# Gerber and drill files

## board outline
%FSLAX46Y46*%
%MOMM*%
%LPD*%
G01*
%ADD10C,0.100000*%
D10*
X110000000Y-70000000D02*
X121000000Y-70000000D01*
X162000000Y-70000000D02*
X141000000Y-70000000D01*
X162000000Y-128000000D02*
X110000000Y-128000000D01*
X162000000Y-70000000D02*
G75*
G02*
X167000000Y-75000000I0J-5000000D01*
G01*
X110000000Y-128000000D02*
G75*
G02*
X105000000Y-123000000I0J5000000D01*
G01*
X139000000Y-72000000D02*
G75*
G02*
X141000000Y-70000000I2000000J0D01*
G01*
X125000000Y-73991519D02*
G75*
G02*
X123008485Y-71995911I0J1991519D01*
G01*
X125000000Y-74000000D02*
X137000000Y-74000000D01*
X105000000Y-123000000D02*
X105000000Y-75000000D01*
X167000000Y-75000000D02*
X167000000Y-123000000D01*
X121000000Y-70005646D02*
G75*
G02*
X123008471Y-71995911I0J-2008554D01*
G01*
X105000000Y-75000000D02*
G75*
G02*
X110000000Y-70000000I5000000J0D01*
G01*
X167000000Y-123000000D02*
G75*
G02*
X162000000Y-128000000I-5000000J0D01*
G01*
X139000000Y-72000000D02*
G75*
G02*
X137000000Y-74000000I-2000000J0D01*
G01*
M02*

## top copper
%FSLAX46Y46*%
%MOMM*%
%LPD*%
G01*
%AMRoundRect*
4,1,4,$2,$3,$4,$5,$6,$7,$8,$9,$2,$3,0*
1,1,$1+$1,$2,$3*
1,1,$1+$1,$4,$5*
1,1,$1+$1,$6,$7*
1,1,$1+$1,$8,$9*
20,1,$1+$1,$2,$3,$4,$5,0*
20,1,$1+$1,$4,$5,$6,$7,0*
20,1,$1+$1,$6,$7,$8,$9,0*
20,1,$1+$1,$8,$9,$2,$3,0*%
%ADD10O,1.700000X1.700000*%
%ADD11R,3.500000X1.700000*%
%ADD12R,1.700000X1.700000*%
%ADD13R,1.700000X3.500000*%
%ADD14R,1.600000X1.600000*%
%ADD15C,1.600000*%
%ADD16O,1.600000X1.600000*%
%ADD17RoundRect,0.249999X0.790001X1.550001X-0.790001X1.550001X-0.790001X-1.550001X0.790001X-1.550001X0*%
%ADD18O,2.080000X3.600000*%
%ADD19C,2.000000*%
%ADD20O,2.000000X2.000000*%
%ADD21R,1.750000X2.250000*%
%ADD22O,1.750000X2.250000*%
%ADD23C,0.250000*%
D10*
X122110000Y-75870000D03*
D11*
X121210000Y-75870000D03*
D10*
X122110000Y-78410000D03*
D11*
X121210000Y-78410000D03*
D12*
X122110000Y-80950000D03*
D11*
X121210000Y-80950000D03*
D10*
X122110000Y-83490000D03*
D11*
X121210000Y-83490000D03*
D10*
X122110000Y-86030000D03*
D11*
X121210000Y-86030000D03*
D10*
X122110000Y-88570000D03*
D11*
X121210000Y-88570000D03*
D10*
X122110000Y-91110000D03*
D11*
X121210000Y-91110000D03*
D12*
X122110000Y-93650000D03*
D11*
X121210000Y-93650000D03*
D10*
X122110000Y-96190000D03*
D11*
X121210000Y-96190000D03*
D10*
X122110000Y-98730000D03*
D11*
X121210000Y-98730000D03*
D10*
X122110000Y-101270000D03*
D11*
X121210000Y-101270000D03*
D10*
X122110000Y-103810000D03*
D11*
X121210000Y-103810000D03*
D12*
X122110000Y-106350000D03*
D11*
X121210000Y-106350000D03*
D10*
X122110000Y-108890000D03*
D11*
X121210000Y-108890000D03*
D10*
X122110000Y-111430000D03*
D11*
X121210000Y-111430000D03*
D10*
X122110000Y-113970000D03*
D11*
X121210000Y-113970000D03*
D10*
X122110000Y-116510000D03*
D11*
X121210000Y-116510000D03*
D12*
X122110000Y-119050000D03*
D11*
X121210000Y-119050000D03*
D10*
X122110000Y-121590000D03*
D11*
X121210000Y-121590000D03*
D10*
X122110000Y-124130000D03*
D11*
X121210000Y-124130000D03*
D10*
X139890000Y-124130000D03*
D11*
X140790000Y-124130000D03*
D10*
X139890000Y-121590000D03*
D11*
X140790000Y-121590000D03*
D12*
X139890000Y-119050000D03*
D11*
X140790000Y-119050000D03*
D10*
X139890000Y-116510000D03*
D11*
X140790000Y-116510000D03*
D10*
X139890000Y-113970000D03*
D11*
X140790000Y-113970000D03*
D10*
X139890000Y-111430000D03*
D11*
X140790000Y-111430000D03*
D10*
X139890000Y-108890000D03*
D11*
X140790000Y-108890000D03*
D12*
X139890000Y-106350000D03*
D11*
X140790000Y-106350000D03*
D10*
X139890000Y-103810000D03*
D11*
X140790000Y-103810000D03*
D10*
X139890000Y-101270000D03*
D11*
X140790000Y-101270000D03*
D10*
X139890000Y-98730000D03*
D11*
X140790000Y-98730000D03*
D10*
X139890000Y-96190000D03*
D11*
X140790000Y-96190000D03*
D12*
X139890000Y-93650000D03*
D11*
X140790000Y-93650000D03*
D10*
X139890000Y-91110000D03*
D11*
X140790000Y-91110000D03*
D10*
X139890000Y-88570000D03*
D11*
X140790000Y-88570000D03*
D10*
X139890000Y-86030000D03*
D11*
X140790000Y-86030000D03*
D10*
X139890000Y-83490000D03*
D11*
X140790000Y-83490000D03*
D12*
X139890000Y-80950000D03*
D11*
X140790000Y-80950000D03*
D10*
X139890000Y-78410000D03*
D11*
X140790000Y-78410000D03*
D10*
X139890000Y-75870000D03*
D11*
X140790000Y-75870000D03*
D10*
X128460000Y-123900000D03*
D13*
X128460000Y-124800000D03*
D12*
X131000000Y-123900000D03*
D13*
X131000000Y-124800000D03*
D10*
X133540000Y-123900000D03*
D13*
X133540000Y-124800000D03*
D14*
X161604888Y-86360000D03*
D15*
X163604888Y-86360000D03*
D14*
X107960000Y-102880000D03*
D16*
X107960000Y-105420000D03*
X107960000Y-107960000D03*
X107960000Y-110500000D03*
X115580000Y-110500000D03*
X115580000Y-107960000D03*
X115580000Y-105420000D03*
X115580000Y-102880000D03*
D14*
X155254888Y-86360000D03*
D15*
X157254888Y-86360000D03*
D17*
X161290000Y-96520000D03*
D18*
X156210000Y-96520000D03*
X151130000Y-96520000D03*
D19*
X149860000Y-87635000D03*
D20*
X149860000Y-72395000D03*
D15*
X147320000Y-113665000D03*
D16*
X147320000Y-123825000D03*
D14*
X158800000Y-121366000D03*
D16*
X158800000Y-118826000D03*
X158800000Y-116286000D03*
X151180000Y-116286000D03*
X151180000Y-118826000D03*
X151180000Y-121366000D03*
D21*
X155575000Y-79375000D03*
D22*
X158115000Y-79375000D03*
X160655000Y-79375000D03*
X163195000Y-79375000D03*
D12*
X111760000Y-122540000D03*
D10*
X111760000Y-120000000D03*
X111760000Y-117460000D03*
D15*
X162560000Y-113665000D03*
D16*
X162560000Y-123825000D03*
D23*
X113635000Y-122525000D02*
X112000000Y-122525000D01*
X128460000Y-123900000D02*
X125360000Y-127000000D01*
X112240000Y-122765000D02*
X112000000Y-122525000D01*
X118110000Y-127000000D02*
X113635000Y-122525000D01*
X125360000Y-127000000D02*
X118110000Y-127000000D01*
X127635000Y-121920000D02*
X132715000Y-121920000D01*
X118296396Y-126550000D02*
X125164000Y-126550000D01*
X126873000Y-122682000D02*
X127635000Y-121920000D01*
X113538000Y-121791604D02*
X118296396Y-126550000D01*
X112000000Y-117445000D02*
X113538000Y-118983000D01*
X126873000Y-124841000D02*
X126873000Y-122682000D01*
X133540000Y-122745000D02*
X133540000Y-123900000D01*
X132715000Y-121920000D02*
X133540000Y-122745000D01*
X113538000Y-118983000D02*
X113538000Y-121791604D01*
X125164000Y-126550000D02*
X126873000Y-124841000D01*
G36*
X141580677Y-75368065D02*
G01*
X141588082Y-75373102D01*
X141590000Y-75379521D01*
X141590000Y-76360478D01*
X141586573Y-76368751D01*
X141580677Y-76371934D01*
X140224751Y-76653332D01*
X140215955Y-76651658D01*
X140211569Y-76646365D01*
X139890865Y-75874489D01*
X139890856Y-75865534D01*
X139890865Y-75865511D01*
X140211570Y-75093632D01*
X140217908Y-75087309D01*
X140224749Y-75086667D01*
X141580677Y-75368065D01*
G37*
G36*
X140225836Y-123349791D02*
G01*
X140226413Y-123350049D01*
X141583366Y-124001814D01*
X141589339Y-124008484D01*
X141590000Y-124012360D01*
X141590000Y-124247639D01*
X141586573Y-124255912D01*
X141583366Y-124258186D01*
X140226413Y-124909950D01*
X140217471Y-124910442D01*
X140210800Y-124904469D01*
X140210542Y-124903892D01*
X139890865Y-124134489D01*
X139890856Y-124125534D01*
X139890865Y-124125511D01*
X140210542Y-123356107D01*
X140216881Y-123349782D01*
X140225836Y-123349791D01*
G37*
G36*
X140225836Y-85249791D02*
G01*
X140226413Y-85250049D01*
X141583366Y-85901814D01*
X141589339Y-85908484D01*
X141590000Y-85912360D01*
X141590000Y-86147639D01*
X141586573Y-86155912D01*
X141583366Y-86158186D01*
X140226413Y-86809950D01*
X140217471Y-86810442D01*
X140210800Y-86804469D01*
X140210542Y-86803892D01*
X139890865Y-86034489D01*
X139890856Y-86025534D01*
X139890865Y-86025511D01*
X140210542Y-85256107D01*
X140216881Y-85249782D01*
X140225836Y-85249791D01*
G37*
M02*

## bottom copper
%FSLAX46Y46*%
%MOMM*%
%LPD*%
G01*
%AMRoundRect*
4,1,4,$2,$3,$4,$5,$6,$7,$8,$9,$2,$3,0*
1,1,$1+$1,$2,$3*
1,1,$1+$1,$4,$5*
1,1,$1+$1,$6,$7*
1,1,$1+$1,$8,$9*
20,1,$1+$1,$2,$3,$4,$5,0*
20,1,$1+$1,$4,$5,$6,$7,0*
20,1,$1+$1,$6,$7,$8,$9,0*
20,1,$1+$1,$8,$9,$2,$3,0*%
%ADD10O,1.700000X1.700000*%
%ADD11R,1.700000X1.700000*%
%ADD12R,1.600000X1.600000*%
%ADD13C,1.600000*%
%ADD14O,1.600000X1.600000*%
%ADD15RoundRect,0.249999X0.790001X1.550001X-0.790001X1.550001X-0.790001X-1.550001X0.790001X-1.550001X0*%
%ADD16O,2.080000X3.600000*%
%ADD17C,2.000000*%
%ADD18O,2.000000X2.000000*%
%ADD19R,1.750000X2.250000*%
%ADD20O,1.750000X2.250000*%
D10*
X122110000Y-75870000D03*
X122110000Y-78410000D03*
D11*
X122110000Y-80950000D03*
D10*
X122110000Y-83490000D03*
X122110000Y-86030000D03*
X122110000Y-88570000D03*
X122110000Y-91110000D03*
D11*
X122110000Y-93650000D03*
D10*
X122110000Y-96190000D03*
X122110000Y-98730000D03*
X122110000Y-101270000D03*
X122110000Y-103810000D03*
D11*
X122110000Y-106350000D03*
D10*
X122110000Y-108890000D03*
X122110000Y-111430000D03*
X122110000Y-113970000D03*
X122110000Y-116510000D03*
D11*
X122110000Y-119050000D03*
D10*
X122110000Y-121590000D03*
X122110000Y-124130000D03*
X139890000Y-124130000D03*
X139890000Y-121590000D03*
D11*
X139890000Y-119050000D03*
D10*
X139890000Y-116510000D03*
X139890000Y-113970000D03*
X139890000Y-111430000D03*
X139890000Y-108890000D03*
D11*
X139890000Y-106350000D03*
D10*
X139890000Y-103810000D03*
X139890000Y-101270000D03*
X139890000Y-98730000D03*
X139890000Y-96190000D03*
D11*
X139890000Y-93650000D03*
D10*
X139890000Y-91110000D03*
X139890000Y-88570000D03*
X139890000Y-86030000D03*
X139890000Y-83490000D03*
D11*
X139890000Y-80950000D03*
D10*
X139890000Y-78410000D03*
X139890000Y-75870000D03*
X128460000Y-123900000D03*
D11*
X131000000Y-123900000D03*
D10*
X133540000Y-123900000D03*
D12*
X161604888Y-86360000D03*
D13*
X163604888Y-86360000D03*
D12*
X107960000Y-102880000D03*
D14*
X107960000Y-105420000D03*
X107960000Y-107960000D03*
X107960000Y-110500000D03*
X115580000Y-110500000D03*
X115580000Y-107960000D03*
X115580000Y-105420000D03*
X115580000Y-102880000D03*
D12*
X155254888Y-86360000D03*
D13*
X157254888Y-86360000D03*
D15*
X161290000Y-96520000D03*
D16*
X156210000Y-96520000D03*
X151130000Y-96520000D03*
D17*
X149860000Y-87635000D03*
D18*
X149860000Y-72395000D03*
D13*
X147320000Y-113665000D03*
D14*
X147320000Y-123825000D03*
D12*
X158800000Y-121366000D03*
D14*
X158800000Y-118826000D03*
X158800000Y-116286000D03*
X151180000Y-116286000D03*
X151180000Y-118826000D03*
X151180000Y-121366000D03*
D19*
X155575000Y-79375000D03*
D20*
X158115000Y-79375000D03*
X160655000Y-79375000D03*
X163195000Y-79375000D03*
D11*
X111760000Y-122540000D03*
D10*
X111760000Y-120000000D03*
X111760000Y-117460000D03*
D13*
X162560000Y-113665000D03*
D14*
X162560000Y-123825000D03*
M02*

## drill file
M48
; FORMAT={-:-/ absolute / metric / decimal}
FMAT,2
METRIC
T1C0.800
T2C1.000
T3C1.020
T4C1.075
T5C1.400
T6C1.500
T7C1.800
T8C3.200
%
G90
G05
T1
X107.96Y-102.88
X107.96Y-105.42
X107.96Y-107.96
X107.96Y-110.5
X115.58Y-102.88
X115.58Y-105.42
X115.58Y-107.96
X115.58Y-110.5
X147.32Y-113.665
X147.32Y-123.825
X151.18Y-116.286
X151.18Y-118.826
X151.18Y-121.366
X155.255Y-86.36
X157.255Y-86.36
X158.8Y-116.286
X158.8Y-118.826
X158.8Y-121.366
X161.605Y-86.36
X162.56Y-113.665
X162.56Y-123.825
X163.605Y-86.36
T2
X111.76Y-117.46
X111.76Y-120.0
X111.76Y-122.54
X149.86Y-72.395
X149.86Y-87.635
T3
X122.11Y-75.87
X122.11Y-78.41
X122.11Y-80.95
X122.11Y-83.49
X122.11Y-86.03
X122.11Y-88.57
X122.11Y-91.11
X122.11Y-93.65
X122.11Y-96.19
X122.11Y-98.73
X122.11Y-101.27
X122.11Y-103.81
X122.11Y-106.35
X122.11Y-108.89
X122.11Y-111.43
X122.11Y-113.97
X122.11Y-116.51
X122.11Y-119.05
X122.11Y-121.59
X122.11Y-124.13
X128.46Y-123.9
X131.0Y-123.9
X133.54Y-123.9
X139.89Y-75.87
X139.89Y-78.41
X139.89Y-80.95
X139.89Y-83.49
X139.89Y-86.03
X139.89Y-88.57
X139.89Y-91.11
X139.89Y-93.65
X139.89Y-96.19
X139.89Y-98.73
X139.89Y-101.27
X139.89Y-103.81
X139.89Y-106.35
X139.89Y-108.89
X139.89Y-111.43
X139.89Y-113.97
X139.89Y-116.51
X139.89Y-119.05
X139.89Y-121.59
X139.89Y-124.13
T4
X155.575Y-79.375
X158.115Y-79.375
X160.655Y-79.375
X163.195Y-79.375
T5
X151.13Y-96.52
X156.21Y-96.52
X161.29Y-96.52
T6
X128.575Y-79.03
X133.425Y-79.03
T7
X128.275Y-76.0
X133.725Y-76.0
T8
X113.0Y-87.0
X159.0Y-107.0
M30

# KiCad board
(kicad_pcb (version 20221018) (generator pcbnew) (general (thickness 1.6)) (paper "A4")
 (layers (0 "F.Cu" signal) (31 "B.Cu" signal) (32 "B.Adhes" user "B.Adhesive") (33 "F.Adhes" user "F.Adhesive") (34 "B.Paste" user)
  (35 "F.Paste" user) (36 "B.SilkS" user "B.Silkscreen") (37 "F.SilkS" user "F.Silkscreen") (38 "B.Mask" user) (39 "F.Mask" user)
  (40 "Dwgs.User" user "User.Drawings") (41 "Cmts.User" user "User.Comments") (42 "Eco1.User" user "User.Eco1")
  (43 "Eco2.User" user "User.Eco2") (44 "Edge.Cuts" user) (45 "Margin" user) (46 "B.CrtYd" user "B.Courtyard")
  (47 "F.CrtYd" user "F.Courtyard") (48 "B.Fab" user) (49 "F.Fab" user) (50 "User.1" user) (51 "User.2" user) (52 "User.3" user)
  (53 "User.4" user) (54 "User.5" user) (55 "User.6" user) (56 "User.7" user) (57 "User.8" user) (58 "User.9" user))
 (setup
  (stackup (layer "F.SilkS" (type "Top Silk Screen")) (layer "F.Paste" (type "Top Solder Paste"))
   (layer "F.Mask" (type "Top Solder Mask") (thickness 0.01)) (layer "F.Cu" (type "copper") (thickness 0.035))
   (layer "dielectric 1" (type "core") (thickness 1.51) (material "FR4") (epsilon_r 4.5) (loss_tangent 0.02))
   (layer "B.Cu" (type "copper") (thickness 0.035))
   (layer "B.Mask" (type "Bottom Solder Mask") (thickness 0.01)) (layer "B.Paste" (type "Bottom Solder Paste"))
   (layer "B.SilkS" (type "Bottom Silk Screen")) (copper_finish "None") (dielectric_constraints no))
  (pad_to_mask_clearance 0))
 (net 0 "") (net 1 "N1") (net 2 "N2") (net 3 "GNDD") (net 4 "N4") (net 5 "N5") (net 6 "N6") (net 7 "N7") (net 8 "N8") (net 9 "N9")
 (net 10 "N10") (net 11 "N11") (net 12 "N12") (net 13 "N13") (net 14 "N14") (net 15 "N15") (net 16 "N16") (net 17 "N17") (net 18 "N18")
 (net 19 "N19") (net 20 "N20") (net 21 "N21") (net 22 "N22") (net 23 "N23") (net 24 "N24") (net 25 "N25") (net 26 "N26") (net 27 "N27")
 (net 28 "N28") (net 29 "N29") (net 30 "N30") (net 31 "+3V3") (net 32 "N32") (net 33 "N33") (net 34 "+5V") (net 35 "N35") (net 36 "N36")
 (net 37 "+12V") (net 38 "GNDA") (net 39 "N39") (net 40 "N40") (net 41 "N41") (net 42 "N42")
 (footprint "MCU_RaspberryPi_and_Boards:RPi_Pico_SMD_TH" (layer "F.Cu") (at 131 100)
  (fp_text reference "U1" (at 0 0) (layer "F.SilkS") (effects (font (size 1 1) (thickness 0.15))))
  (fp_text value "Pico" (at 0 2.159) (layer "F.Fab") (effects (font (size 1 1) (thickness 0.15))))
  (pad "" np_thru_hole oval (at -2.725 -24) (size 1.8 1.8) (drill 1.8) (layers "*.Cu" "*.Mask"))
  (pad "" np_thru_hole oval (at -2.425 -20.97) (size 1.5 1.5) (drill 1.5) (layers "*.Cu" "*.Mask"))
  (pad "" np_thru_hole oval (at 2.425 -20.97) (size 1.5 1.5) (drill 1.5) (layers "*.Cu" "*.Mask"))
  (pad "" np_thru_hole oval (at 2.725 -24) (size 1.8 1.8) (drill 1.8) (layers "*.Cu" "*.Mask"))
  (pad "1" thru_hole oval (at -8.89 -24.13) (size 1.7 1.7) (drill 1.02) (layers "*.Cu" "*.Mask") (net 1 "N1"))
  (pad "1" smd rect (at -8.89 -24.13) (size 3.5 1.7) (drill (offset -0.9 0)) (layers "F.Cu" "F.Mask") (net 1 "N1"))
  (pad "2" thru_hole oval (at -8.89 -21.59) (size 1.7 1.7) (drill 1.02) (layers "*.Cu" "*.Mask") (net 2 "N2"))
  (pad "2" smd rect (at -8.89 -21.59) (size 3.5 1.7) (drill (offset -0.9 0)) (layers "F.Cu" "F.Mask") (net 2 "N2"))
  (pad "3" thru_hole rect (at -8.89 -19.05) (size 1.7 1.7) (drill 1.02) (layers "*.Cu" "*.Mask") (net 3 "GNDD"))
  (pad "3" smd rect (at -8.89 -19.05) (size 3.5 1.7) (drill (offset -0.9 0)) (layers "F.Cu" "F.Mask") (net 3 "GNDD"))
  (pad "4" thru_hole oval (at -8.89 -16.51) (size 1.7 1.7) (drill 1.02) (layers "*.Cu" "*.Mask") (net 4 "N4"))
  (pad "4" smd rect (at -8.89 -16.51) (size 3.5 1.7) (drill (offset -0.9 0)) (layers "F.Cu" "F.Mask") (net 4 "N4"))
  (pad "5" thru_hole oval (at -8.89 -13.97) (size 1.7 1.7) (drill 1.02) (layers "*.Cu" "*.Mask") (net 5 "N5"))
  (pad "5" smd rect (at -8.89 -13.97) (size 3.5 1.7) (drill (offset -0.9 0)) (layers "F.Cu" "F.Mask") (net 5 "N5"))
  (pad "6" thru_hole oval (at -8.89 -11.43) (size 1.7 1.7) (drill 1.02) (layers "*.Cu" "*.Mask") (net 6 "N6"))
  (pad "6" smd rect (at -8.89 -11.43) (size 3.5 1.7) (drill (offset -0.9 0)) (layers "F.Cu" "F.Mask") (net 6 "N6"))
  (pad "7" thru_hole oval (at -8.89 -8.89) (size 1.7 1.7) (drill 1.02) (layers "*.Cu" "*.Mask") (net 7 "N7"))
  (pad "7" smd rect (at -8.89 -8.89) (size 3.5 1.7) (drill (offset -0.9 0)) (layers "F.Cu" "F.Mask") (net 7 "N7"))
  (pad "8" thru_hole rect (at -8.89 -6.35) (size 1.7 1.7) (drill 1.02) (layers "*.Cu" "*.Mask") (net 3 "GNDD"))
  (pad "8" smd rect (at -8.89 -6.35) (size 3.5 1.7) (drill (offset -0.9 0)) (layers "F.Cu" "F.Mask") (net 3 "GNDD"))
  (pad "9" thru_hole oval (at -8.89 -3.81) (size 1.7 1.7) (drill 1.02) (layers "*.Cu" "*.Mask") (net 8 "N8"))
  (pad "9" smd rect (at -8.89 -3.81) (size 3.5 1.7) (drill (offset -0.9 0)) (layers "F.Cu" "F.Mask") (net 8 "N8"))
  (pad "10" thru_hole oval (at -8.89 -1.27) (size 1.7 1.7) (drill 1.02) (layers "*.Cu" "*.Mask") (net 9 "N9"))
  (pad "10" smd rect (at -8.89 -1.27) (size 3.5 1.7) (drill (offset -0.9 0)) (layers "F.Cu" "F.Mask") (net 9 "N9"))
  (pad "11" thru_hole oval (at -8.89 1.27) (size 1.7 1.7) (drill 1.02) (layers "*.Cu" "*.Mask") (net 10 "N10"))
  (pad "11" smd rect (at -8.89 1.27) (size 3.5 1.7) (drill (offset -0.9 0)) (layers "F.Cu" "F.Mask") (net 10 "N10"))
  (pad "12" thru_hole oval (at -8.89 3.81) (size 1.7 1.7) (drill 1.02) (layers "*.Cu" "*.Mask") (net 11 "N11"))
  (pad "12" smd rect (at -8.89 3.81) (size 3.5 1.7) (drill (offset -0.9 0)) (layers "F.Cu" "F.Mask") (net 11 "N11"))
  (pad "13" thru_hole rect (at -8.89 6.35) (size 1.7 1.7) (drill 1.02) (layers "*.Cu" "*.Mask") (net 3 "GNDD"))
  (pad "13" smd rect (at -8.89 6.35) (size 3.5 1.7) (drill (offset -0.9 0)) (layers "F.Cu" "F.Mask") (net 3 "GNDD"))
  (pad "14" thru_hole oval (at -8.89 8.89) (size 1.7 1.7) (drill 1.02) (layers "*.Cu" "*.Mask") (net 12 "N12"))
  (pad "14" smd rect (at -8.89 8.89) (size 3.5 1.7) (drill (offset -0.9 0)) (layers "F.Cu" "F.Mask") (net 12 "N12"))
  (pad "15" thru_hole oval (at -8.89 11.43) (size 1.7 1.7) (drill 1.02) (layers "*.Cu" "*.Mask") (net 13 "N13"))
  (pad "15" smd rect (at -8.89 11.43) (size 3.5 1.7) (drill (offset -0.9 0)) (layers "F.Cu" "F.Mask") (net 13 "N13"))
  (pad "16" thru_hole oval (at -8.89 13.97) (size 1.7 1.7) (drill 1.02) (layers "*.Cu" "*.Mask") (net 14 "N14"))
  (pad "16" smd rect (at -8.89 13.97) (size 3.5 1.7) (drill (offset -0.9 0)) (layers "F.Cu" "F.Mask") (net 14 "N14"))
  (pad "17" thru_hole oval (at -8.89 16.51) (size 1.7 1.7) (drill 1.02) (layers "*.Cu" "*.Mask") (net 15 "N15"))
  (pad "17" smd rect (at -8.89 16.51) (size 3.5 1.7) (drill (offset -0.9 0)) (layers "F.Cu" "F.Mask") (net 15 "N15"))
  (pad "18" thru_hole rect (at -8.89 19.05) (size 1.7 1.7) (drill 1.02) (layers "*.Cu" "*.Mask") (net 3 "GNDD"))
  (pad "18" smd rect (at -8.89 19.05) (size 3.5 1.7) (drill (offset -0.9 0)) (layers "F.Cu" "F.Mask") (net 3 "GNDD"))
  (pad "19" thru_hole oval (at -8.89 21.59) (size 1.7 1.7) (drill 1.02) (layers "*.Cu" "*.Mask") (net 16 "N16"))
  (pad "19" smd rect (at -8.89 21.59) (size 3.5 1.7) (drill (offset -0.9 0)) (layers "F.Cu" "F.Mask") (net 16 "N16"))
  (pad "20" thru_hole oval (at -8.89 24.13) (size 1.7 1.7) (drill 1.02) (layers "*.Cu" "*.Mask") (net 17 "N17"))
  (pad "20" smd rect (at -8.89 24.13) (size 3.5 1.7) (drill (offset -0.9 0)) (layers "F.Cu" "F.Mask") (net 17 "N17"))
  (pad "21" thru_hole oval (at 8.89 24.13) (size 1.7 1.7) (drill 1.02) (layers "*.Cu" "*.Mask") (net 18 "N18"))
  (pad "21" smd rect (at 8.89 24.13) (size 3.5 1.7) (drill (offset 0.9 0)) (layers "F.Cu" "F.Mask") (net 18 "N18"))
  (pad "22" thru_hole oval (at 8.89 21.59) (size 1.7 1.7) (drill 1.02) (layers "*.Cu" "*.Mask") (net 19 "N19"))
  (pad "22" smd rect (at 8.89 21.59) (size 3.5 1.7) (drill (offset 0.9 0)) (layers "F.Cu" "F.Mask") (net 19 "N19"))
  (pad "23" thru_hole rect (at 8.89 19.05) (size 1.7 1.7) (drill 1.02) (layers "*.Cu" "*.Mask") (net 3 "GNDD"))
  (pad "23" smd rect (at 8.89 19.05) (size 3.5 1.7) (drill (offset 0.9 0)) (layers "F.Cu" "F.Mask") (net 3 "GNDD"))
  (pad "24" thru_hole oval (at 8.89 16.51) (size 1.7 1.7) (drill 1.02) (layers "*.Cu" "*.Mask") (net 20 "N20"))
  (pad "24" smd rect (at 8.89 16.51) (size 3.5 1.7) (drill (offset 0.9 0)) (layers "F.Cu" "F.Mask") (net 20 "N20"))
  (pad "25" thru_hole oval (at 8.89 13.97) (size 1.7 1.7) (drill 1.02) (layers "*.Cu" "*.Mask") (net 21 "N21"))
  (pad "25" smd rect (at 8.89 13.97) (size 3.5 1.7) (drill (offset 0.9 0)) (layers "F.Cu" "F.Mask") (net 21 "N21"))
  (pad "26" thru_hole oval (at 8.89 11.43) (size 1.7 1.7) (drill 1.02) (layers "*.Cu" "*.Mask") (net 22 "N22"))
  (pad "26" smd rect (at 8.89 11.43) (size 3.5 1.7) (drill (offset 0.9 0)) (layers "F.Cu" "F.Mask") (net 22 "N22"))
  (pad "27" thru_hole oval (at 8.89 8.89) (size 1.7 1.7) (drill 1.02) (layers "*.Cu" "*.Mask") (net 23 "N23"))
  (pad "27" smd rect (at 8.89 8.89) (size 3.5 1.7) (drill (offset 0.9 0)) (layers "F.Cu" "F.Mask") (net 23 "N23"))
  (pad "28" thru_hole rect (at 8.89 6.35) (size 1.7 1.7) (drill 1.02) (layers "*.Cu" "*.Mask") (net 3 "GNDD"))
  (pad "28" smd rect (at 8.89 6.35) (size 3.5 1.7) (drill (offset 0.9 0)) (layers "F.Cu" "F.Mask") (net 3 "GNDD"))
  (pad "29" thru_hole oval (at 8.89 3.81) (size 1.7 1.7) (drill 1.02) (layers "*.Cu" "*.Mask") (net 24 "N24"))
  (pad "29" smd rect (at 8.89 3.81) (size 3.5 1.7) (drill (offset 0.9 0)) (layers "F.Cu" "F.Mask") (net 24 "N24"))
  (pad "30" thru_hole oval (at 8.89 1.27) (size 1.7 1.7) (drill 1.02) (layers "*.Cu" "*.Mask") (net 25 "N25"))
  (pad "30" smd rect (at 8.89 1.27) (size 3.5 1.7) (drill (offset 0.9 0)) (layers "F.Cu" "F.Mask") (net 25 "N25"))
  (pad "31" thru_hole oval (at 8.89 -1.27) (size 1.7 1.7) (drill 1.02) (layers "*.Cu" "*.Mask") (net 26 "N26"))
  (pad "31" smd rect (at 8.89 -1.27) (size 3.5 1.7) (drill (offset 0.9 0)) (layers "F.Cu" "F.Mask") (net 26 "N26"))
  (pad "32" thru_hole oval (at 8.89 -3.81) (size 1.7 1.7) (drill 1.02) (layers "*.Cu" "*.Mask") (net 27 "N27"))
  (pad "32" smd rect (at 8.89 -3.81) (size 3.5 1.7) (drill (offset 0.9 0)) (layers "F.Cu" "F.Mask") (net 27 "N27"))
  (pad "33" thru_hole rect (at 8.89 -6.35) (size 1.7 1.7) (drill 1.02) (layers "*.Cu" "*.Mask") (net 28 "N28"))
  (pad "33" smd rect (at 8.89 -6.35) (size 3.5 1.7) (drill (offset 0.9 0)) (layers "F.Cu" "F.Mask") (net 28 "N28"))
  (pad "34" thru_hole oval (at 8.89 -8.89) (size 1.7 1.7) (drill 1.02) (layers "*.Cu" "*.Mask") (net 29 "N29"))
  (pad "34" smd rect (at 8.89 -8.89) (size 3.5 1.7) (drill (offset 0.9 0)) (layers "F.Cu" "F.Mask") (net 29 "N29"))
  (pad "35" thru_hole oval (at 8.89 -11.43) (size 1.7 1.7) (drill 1.02) (layers "*.Cu" "*.Mask") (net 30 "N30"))
  (pad "35" smd rect (at 8.89 -11.43) (size 3.5 1.7) (drill (offset 0.9 0)) (layers "F.Cu" "F.Mask") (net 30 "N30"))
  (pad "36" thru_hole oval (at 8.89 -13.97) (size 1.7 1.7) (drill 1.02) (layers "*.Cu" "*.Mask") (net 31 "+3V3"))
  (pad "36" smd rect (at 8.89 -13.97) (size 3.5 1.7) (drill (offset 0.9 0)) (layers "F.Cu" "F.Mask") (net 31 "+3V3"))
  (pad "37" thru_hole oval (at 8.89 -16.51) (size 1.7 1.7) (drill 1.02) (layers "*.Cu" "*.Mask") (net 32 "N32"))
  (pad "37" smd rect (at 8.89 -16.51) (size 3.5 1.7) (drill (offset 0.9 0)) (layers "F.Cu" "F.Mask") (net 32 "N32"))
  (pad "38" thru_hole rect (at 8.89 -19.05) (size 1.7 1.7) (drill 1.02) (layers "*.Cu" "*.Mask") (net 3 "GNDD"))
  (pad "38" smd rect (at 8.89 -19.05) (size 3.5 1.7) (drill (offset 0.9 0)) (layers "F.Cu" "F.Mask") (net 3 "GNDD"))
  (pad "39" thru_hole oval (at 8.89 -21.59) (size 1.7 1.7) (drill 1.02) (layers "*.Cu" "*.Mask") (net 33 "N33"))
  (pad "39" smd rect (at 8.89 -21.59) (size 3.5 1.7) (drill (offset 0.9 0)) (layers "F.Cu" "F.Mask") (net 33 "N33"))
  (pad "40" thru_hole oval (at 8.89 -24.13) (size 1.7 1.7) (drill 1.02) (layers "*.Cu" "*.Mask") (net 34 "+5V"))
  (pad "40" smd rect (at 8.89 -24.13) (size 3.5 1.7) (drill (offset 0.9 0)) (layers "F.Cu" "F.Mask") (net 34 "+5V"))
  (pad "41" thru_hole oval (at -2.54 23.9) (size 1.7 1.7) (drill 1.02) (layers "*.Cu" "*.Mask") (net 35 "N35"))
  (pad "41" smd rect (at -2.54 23.9 90) (size 3.5 1.7) (drill (offset -0.9 0)) (layers "F.Cu" "F.Mask") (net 35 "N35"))
  (pad "42" thru_hole rect (at 0 23.9) (size 1.7 1.7) (drill 1.02) (layers "*.Cu" "*.Mask") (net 3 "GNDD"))
  (pad "42" smd rect (at 0 23.9 90) (size 3.5 1.7) (drill (offset -0.9 0)) (layers "F.Cu" "F.Mask") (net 3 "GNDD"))
  (pad "43" thru_hole oval (at 2.54 23.9) (size 1.7 1.7) (drill 1.02) (layers "*.Cu" "*.Mask") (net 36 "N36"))
  (pad "43" smd rect (at 2.54 23.9 90) (size 3.5 1.7) (drill (offset -0.9 0)) (layers "F.Cu" "F.Mask") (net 36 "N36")))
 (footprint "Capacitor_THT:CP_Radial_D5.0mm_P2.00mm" (layer "F.Cu") (at 161.604888 86.36)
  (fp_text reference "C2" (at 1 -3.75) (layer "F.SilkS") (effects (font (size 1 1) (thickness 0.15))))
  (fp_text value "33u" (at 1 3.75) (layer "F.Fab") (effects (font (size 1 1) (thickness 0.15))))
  (pad "1" thru_hole rect (at 0 0) (size 1.6 1.6) (drill 0.8) (layers "*.Cu" "*.Mask") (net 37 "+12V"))
  (pad "2" thru_hole circle (at 2 0) (size 1.6 1.6) (drill 0.8) (layers "*.Cu" "*.Mask") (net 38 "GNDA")))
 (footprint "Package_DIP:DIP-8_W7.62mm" (layer "F.Cu") (at 107.96 102.88)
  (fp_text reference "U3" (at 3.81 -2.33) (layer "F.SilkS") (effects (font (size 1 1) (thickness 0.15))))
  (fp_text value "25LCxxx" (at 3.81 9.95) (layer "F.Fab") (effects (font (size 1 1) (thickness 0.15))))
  (pad "1" thru_hole rect (at 0 0) (size 1.6 1.6) (drill 0.8) (layers "*.Cu" "*.Mask") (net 9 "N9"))
  (pad "2" thru_hole oval (at 0 2.54) (size 1.6 1.6) (drill 0.8) (layers "*.Cu" "*.Mask") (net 10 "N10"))
  (pad "3" thru_hole oval (at 0 5.08) (size 1.6 1.6) (drill 0.8) (layers "*.Cu" "*.Mask") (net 14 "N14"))
  (pad "4" thru_hole oval (at 0 7.62) (size 1.6 1.6) (drill 0.8) (layers "*.Cu" "*.Mask") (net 3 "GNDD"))
  (pad "5" thru_hole oval (at 7.62 7.62) (size 1.6 1.6) (drill 0.8) (layers "*.Cu" "*.Mask") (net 13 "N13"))
  (pad "6" thru_hole oval (at 7.62 5.08) (size 1.6 1.6) (drill 0.8) (layers "*.Cu" "*.Mask") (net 12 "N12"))
  (pad "7" thru_hole oval (at 7.62 2.54) (size 1.6 1.6) (drill 0.8) (layers "*.Cu" "*.Mask") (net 11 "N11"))
  (pad "8" thru_hole oval (at 7.62 0) (size 1.6 1.6) (drill 0.8) (layers "*.Cu" "*.Mask") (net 31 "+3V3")))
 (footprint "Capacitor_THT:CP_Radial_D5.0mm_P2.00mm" (layer "F.Cu") (at 155.254888 86.36)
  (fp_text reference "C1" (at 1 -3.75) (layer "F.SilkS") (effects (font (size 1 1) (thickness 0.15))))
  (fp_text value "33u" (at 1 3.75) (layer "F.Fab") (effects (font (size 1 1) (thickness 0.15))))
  (pad "1" thru_hole rect (at 0 0) (size 1.6 1.6) (drill 0.8) (layers "*.Cu" "*.Mask") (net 34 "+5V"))
  (pad "2" thru_hole circle (at 2 0) (size 1.6 1.6) (drill 0.8) (layers "*.Cu" "*.Mask") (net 3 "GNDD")))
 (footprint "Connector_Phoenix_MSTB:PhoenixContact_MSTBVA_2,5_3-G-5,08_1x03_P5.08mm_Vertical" (layer "F.Cu") (at 161.29 96.52 180)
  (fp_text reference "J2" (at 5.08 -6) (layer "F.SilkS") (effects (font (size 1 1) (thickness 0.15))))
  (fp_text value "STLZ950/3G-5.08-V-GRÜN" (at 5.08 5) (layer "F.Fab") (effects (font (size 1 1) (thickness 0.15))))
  (pad "1" thru_hole roundrect (at 0 0 180) (size 2.08 3.6) (drill 1.4) (layers "*.Cu" "*.Mask") (roundrect_rratio 0.120192) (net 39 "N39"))
  (pad "2" thru_hole oval (at 5.08 0 180) (size 2.08 3.6) (drill 1.4) (layers "*.Cu" "*.Mask") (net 38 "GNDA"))
  (pad "3" thru_hole oval (at 10.16 0 180) (size 2.08 3.6) (drill 1.4) (layers "*.Cu" "*.Mask") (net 37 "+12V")))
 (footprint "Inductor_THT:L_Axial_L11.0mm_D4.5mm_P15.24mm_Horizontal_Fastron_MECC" (layer "F.Cu") (at 149.86 87.635 90)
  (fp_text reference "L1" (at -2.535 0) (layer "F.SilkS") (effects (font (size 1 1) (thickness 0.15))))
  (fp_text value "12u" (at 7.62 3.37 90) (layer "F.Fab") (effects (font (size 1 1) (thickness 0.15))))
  (pad "1" thru_hole circle (at 0 0 90) (size 2 2) (drill 1) (layers "*.Cu" "*.Mask") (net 34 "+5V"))
  (pad "2" thru_hole oval (at 15.24 0 90) (size 2 2) (drill 1) (layers "*.Cu" "*.Mask") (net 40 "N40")))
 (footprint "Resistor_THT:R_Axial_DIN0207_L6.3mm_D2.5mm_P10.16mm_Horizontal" (layer "F.Cu") (at 147.32 113.665 -90)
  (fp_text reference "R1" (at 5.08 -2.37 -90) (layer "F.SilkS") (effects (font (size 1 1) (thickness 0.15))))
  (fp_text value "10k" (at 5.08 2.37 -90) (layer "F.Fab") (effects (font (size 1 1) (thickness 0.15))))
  (pad "1" thru_hole circle (at 0 0 270) (size 1.6 1.6) (drill 0.8) (layers "*.Cu" "*.Mask") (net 31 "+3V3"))
  (pad "2" thru_hole oval (at 10.16 0 270) (size 1.6 1.6) (drill 0.8) (layers "*.Cu" "*.Mask") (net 18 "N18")))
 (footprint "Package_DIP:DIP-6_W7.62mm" (layer "F.Cu") (at 158.8 121.366 180)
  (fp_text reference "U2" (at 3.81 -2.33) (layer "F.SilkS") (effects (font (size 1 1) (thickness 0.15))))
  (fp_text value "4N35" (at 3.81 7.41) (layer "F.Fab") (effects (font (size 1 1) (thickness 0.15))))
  (pad "1" thru_hole rect (at 0 0 180) (size 1.6 1.6) (drill 0.8) (layers "*.Cu" "*.Mask") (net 39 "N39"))
  (pad "2" thru_hole oval (at 0 2.54 180) (size 1.6 1.6) (drill 0.8) (layers "*.Cu" "*.Mask") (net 38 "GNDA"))
  (pad "3" thru_hole oval (at 0 5.08 180) (size 1.6 1.6) (drill 0.8) (layers "*.Cu" "*.Mask") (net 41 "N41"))
  (pad "4" thru_hole oval (at 7.62 5.08 180) (size 1.6 1.6) (drill 0.8) (layers "*.Cu" "*.Mask") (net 3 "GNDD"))
  (pad "5" thru_hole oval (at 7.62 2.54 180) (size 1.6 1.6) (drill 0.8) (layers "*.Cu" "*.Mask") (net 18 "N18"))
  (pad "6" thru_hole oval (at 7.62 0 180) (size 1.6 1.6) (drill 0.8) (layers "*.Cu" "*.Mask") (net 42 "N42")))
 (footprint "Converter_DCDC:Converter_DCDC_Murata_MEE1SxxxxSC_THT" (layer "F.Cu") (at 155.575 79.375 90)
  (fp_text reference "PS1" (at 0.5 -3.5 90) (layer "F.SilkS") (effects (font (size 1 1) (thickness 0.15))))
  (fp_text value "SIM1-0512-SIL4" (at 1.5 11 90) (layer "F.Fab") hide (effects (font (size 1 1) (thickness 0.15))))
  (pad "1" thru_hole rect (at 0 0) (size 1.75 2.25) (drill 1.075) (layers "*.Cu" "*.Mask") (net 3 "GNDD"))
  (pad "2" thru_hole oval (at 0 2.54) (size 1.75 2.25) (drill 1.075) (layers "*.Cu" "*.Mask") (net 40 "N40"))
  (pad "3" thru_hole oval (at 0 5.08) (size 1.75 2.25) (drill 1.075) (layers "*.Cu" "*.Mask") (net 38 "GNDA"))
  (pad "4" thru_hole oval (at 0 7.62) (size 1.75 2.25) (drill 1.075) (layers "*.Cu" "*.Mask") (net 37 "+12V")))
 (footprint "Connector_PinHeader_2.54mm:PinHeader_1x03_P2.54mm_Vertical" (layer "F.Cu") (at 111.76 122.54 180)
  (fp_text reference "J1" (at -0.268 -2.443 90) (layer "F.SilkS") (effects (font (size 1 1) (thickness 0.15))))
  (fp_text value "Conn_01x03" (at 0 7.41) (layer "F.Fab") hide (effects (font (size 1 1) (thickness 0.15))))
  (pad "1" thru_hole rect (at 0 0 180) (size 1.7 1.7) (drill 1) (layers "*.Cu" "*.Mask") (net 35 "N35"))
  (pad "2" thru_hole oval (at 0 2.54 180) (size 1.7 1.7) (drill 1) (layers "*.Cu" "*.Mask") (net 3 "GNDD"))
  (pad "3" thru_hole oval (at 0 5.08 180) (size 1.7 1.7) (drill 1) (layers "*.Cu" "*.Mask") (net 36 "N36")))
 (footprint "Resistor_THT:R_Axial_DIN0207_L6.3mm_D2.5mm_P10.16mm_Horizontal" (layer "F.Cu") (at 162.56 113.665 -90)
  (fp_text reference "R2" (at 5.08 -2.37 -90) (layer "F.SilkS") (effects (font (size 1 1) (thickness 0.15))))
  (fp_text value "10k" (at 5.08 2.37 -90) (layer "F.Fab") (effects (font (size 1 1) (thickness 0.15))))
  (pad "1" thru_hole circle (at 0 0 270) (size 1.6 1.6) (drill 0.8) (layers "*.Cu" "*.Mask") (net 37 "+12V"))
  (pad "2" thru_hole oval (at 10.16 0 270) (size 1.6 1.6) (drill 0.8) (layers "*.Cu" "*.Mask") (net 39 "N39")))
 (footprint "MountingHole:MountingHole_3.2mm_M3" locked (layer "F.Cu") (at 159 107)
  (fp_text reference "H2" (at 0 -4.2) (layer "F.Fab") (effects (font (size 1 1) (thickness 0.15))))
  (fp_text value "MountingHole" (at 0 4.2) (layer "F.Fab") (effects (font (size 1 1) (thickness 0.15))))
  (pad "" np_thru_hole circle locked (at 0 0) (size 3.2 3.2) (drill 3.2) (layers "*.Cu" "*.Mask")))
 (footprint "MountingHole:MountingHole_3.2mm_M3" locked (layer "F.Cu") (at 113 87)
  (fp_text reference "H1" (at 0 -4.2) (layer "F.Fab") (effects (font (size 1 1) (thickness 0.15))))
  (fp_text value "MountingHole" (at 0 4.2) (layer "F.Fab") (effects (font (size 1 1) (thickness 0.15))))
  (pad "" np_thru_hole circle locked (at 0 0) (size 3.2 3.2) (drill 3.2) (layers "*.Cu" "*.Mask")))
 (gr_line (start 110 70) (end 121 70) (stroke (width 0.1) (type default)) (layer "Edge.Cuts"))
 (gr_line (start 162 70) (end 141 70) (stroke (width 0.1) (type default)) (layer "Edge.Cuts"))
 (gr_line (start 162 128) (end 110 128) (stroke (width 0.1) (type default)) (layer "Edge.Cuts"))
 (gr_arc (start 162 70) (mid 165.535534 71.464466) (end 167 75) (stroke (width 0.1) (type default)) (layer "Edge.Cuts"))
 (gr_arc (start 110 128) (mid 106.464466 126.535534) (end 105 123) (stroke (width 0.1) (type default)) (layer "Edge.Cuts"))
 (gr_arc (start 139 72) (mid 139.585786 70.585786) (end 141 70) (stroke (width 0.1) (type default)) (layer "Edge.Cuts"))
 (gr_arc (start 125 73.991519) (mid 123.590338 73.40677) (end 123.008485 71.995911) (stroke (width 0.1) (type default)) (layer "Edge.Cuts"))
 (gr_line (start 125 74) (end 137 74) (stroke (width 0.1) (type default)) (layer "Edge.Cuts"))
 (gr_line (start 105 123) (end 105 75) (stroke (width 0.1) (type default)) (layer "Edge.Cuts"))
 (gr_line (start 167 75) (end 167 123) (stroke (width 0.1) (type default)) (layer "Edge.Cuts"))
 (gr_arc (start 121 70.005646) (mid 122.413786 70.587486) (end 123.008485 71.995911) (stroke (width 0.1) (type default)) (layer "Edge.Cuts"))
 (gr_arc (start 105 75) (mid 106.464466 71.464466) (end 110 70) (stroke (width 0.1) (type default)) (layer "Edge.Cuts"))
 (gr_arc (start 167 123) (mid 165.535534 126.535534) (end 162 128) (stroke (width 0.1) (type default)) (layer "Edge.Cuts"))
 (gr_arc (start 139 72) (mid 138.414214 73.414214) (end 137 74) (stroke (width 0.1) (type default)) (layer "Edge.Cuts"))
 (segment (start 113.635 122.525) (end 112 122.525) (width 0.25) (layer "F.Cu") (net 35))
 (segment (start 128.46 123.9) (end 125.36 127) (width 0.25) (layer "F.Cu") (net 35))
 (segment (start 112.24 122.765) (end 112 122.525) (width 0.25) (layer "F.Cu") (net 35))
 (segment (start 118.11 127) (end 113.635 122.525) (width 0.25) (layer "F.Cu") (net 35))
 (segment (start 125.36 127) (end 118.11 127) (width 0.25) (layer "F.Cu") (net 35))
 (segment (start 127.635 121.92) (end 132.715 121.92) (width 0.25) (layer "F.Cu") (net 36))
 (segment (start 118.296396 126.55) (end 125.164 126.55) (width 0.25) (layer "F.Cu") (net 36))
 (segment (start 126.873 122.682) (end 127.635 121.92) (width 0.25) (layer "F.Cu") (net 36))
 (segment (start 113.538 121.791604) (end 118.296396 126.55) (width 0.25) (layer "F.Cu") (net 36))
 (segment (start 112 117.445) (end 113.538 118.983) (width 0.25) (layer "F.Cu") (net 36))
 (segment (start 126.873 124.841) (end 126.873 122.682) (width 0.25) (layer "F.Cu") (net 36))
 (segment (start 133.54 122.745) (end 133.54 123.9) (width 0.25) (layer "F.Cu") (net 36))
 (segment (start 132.715 121.92) (end 133.54 122.745) (width 0.25) (layer "F.Cu") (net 36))
 (segment (start 113.538 118.983) (end 113.538 121.791604) (width 0.25) (layer "F.Cu") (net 36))
 (segment (start 125.164 126.55) (end 126.873 124.841) (width 0.25) (layer "F.Cu") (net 36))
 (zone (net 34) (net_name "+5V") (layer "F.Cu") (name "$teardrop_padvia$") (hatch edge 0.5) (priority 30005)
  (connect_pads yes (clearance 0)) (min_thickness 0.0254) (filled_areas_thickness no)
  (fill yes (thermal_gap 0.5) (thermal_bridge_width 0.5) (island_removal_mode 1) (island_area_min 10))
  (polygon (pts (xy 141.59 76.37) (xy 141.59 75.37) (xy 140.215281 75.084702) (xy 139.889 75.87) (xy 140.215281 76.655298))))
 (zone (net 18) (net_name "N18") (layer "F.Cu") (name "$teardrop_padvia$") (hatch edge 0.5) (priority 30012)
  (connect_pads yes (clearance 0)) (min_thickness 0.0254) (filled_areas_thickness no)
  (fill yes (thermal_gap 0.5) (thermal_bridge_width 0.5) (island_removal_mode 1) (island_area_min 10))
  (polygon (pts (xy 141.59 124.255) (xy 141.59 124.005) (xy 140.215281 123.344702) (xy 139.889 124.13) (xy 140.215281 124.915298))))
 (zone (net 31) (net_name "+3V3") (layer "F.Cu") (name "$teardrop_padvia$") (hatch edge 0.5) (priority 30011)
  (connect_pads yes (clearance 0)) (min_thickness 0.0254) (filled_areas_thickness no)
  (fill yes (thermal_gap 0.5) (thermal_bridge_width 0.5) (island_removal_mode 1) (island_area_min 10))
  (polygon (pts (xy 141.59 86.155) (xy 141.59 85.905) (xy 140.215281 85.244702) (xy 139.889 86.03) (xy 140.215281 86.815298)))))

